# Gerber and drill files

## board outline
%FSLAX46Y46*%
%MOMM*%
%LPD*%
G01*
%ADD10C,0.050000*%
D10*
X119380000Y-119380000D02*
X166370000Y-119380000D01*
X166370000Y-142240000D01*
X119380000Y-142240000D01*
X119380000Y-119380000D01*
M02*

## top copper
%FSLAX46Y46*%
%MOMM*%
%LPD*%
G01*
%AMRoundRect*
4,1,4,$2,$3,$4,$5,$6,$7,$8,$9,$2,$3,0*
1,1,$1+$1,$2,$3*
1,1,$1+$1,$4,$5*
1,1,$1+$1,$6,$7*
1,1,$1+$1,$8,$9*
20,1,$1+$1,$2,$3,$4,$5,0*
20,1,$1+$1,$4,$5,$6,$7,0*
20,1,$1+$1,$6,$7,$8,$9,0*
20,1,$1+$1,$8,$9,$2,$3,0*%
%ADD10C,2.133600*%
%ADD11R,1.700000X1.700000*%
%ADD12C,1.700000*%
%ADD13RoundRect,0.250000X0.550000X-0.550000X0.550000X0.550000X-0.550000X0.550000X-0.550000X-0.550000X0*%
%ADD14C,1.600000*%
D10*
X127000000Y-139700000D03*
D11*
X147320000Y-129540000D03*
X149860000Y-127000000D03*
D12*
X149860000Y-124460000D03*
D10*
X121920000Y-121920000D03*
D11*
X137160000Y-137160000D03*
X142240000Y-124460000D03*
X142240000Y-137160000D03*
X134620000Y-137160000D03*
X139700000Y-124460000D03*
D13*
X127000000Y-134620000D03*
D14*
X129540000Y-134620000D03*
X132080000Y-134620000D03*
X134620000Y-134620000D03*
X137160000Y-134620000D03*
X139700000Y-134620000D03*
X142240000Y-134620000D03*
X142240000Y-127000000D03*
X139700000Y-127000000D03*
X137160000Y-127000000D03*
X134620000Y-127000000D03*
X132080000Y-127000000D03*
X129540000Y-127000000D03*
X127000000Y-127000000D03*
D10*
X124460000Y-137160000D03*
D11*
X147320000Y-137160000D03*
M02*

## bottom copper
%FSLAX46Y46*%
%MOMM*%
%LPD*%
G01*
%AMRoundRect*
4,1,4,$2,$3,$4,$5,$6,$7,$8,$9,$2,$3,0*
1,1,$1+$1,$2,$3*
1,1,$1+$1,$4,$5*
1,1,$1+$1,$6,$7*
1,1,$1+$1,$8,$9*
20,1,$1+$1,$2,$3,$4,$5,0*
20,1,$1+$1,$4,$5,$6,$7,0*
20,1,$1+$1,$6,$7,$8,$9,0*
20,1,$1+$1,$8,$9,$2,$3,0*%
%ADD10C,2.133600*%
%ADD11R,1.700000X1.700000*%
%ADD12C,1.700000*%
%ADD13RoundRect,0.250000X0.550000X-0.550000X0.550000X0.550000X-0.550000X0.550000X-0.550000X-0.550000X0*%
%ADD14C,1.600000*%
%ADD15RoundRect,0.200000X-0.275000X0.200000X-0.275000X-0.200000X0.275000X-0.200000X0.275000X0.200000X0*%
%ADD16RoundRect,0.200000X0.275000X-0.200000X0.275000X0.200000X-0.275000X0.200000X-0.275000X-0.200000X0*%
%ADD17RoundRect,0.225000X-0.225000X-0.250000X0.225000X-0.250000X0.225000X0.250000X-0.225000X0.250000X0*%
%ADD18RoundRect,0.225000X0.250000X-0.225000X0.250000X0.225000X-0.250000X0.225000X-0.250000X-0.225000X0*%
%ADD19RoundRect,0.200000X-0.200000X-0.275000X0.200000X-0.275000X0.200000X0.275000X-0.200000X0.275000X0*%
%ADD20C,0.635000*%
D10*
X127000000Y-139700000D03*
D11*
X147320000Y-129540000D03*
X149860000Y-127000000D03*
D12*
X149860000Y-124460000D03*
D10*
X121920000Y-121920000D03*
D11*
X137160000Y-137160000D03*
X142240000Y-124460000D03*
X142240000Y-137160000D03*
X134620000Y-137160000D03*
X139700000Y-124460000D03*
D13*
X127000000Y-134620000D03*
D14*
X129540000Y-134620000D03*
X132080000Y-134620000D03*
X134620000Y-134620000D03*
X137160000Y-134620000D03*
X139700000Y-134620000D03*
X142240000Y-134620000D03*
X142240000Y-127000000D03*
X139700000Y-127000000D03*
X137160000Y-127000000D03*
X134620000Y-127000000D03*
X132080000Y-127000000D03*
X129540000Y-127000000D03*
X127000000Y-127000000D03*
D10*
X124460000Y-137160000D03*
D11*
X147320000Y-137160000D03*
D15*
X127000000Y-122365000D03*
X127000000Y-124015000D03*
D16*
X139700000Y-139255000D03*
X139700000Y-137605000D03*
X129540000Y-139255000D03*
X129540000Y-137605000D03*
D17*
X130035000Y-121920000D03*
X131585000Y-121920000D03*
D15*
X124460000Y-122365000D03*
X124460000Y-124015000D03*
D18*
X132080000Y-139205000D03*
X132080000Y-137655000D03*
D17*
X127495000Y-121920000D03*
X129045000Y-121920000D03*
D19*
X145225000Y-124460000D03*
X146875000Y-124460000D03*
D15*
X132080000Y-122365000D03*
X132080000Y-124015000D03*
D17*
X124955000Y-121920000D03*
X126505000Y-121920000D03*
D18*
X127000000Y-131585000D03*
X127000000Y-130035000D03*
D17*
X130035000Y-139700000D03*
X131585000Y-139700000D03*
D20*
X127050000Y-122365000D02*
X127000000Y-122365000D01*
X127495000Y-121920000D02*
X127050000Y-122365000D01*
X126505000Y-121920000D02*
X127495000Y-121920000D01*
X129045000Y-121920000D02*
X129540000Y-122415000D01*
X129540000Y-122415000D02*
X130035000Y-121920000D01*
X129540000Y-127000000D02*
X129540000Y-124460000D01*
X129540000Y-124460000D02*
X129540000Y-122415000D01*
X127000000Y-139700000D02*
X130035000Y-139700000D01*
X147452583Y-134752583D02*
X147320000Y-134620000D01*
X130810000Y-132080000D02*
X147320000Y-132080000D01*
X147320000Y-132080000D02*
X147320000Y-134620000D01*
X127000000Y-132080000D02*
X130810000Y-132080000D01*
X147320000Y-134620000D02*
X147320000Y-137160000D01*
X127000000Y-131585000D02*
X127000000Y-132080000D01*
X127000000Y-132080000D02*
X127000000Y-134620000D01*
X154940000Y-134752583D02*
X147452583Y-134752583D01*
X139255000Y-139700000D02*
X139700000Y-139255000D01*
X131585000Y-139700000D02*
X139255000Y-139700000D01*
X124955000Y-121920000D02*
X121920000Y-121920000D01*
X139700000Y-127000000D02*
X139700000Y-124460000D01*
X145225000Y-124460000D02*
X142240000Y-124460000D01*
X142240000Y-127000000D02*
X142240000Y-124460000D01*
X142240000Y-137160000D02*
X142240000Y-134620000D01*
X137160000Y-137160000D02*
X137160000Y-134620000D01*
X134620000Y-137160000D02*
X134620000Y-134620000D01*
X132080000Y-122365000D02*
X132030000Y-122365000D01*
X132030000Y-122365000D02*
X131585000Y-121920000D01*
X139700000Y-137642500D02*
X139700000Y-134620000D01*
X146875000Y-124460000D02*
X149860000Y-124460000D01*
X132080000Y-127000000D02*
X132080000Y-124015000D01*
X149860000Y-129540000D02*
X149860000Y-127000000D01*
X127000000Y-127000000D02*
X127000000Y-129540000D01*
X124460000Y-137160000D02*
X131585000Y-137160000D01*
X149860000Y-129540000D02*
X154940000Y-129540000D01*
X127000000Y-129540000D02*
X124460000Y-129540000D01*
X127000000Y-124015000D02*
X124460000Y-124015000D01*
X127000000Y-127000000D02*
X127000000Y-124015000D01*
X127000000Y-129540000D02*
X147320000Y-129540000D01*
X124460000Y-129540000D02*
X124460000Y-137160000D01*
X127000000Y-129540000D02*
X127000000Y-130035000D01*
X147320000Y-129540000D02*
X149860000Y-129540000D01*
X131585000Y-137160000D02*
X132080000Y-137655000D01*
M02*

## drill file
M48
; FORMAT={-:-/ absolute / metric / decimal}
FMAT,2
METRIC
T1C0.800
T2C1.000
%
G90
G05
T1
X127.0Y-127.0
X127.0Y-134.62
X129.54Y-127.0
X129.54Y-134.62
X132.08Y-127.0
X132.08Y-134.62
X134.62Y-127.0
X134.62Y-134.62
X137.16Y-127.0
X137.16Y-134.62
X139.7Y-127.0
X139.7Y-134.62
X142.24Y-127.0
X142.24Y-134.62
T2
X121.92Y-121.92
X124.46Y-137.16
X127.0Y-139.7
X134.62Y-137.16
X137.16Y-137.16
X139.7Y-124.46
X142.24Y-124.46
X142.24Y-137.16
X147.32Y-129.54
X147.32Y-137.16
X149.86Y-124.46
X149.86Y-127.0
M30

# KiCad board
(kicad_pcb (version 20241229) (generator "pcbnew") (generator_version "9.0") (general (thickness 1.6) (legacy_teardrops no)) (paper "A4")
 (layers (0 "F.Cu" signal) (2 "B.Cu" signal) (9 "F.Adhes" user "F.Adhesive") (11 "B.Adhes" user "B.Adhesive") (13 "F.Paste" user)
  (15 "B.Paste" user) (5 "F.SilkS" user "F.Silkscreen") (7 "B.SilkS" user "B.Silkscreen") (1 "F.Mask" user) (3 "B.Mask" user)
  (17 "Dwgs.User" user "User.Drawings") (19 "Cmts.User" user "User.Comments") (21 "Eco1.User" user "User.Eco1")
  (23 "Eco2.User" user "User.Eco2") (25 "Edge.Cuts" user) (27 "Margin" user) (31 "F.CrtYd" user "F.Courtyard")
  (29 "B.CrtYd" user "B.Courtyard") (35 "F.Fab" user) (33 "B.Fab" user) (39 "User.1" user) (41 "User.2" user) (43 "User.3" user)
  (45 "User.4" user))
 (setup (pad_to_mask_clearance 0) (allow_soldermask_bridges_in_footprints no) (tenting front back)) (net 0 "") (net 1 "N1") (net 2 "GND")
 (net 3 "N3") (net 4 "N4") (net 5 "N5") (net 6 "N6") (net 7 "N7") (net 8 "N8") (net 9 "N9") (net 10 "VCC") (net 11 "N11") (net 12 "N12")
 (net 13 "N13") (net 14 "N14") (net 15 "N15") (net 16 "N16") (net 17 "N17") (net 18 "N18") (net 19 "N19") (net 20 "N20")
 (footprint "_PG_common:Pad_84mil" (layer "F.Cu") (at 127 139.7)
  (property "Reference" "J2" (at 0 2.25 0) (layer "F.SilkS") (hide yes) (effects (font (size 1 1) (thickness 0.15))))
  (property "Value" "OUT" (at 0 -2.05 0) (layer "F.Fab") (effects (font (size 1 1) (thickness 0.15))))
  (pad "1" thru_hole circle (at 0 0) (size 2.1336 2.1336) (drill 1) (layers "*.Cu" "*.Mask") (remove_unused_layers no) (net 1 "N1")))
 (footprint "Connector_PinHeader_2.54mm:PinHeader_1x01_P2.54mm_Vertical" (layer "F.Cu") (at 147.32 129.54)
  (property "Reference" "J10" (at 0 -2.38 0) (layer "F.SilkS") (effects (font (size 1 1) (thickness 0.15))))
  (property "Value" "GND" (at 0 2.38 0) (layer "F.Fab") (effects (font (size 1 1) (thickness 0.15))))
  (pad "1" thru_hole rect (at 0 0) (size 1.7 1.7) (drill 1) (layers "*.Cu" "*.Mask") (remove_unused_layers no) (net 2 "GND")))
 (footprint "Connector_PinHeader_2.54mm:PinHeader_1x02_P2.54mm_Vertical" (layer "F.Cu") (at 149.86 127 180)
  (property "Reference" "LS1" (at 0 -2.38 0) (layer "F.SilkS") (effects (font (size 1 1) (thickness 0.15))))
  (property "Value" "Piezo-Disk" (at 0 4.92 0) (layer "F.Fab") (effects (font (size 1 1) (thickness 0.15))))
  (pad "1" thru_hole rect (at 0 0 180) (size 1.7 1.7) (drill 1) (layers "*.Cu" "*.Mask") (remove_unused_layers no) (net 2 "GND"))
  (pad "2" thru_hole circle (at 0 2.54 180) (size 1.7 1.7) (drill 1) (layers "*.Cu" "*.Mask") (remove_unused_layers no) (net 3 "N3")))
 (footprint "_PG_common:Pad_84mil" (layer "F.Cu") (at 121.92 121.92)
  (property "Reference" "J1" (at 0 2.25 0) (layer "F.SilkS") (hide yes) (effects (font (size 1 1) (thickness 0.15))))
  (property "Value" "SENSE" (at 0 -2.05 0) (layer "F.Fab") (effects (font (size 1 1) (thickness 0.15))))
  (pad "1" thru_hole circle (at 0 0) (size 2.1336 2.1336) (drill 1) (layers "*.Cu" "*.Mask") (remove_unused_layers no) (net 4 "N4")))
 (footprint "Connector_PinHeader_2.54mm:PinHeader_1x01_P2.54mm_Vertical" (layer "F.Cu") (at 137.16 137.16)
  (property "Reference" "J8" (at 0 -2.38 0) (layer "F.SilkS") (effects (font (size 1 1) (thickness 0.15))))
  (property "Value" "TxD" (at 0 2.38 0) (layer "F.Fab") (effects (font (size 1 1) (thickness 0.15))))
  (pad "1" thru_hole rect (at 0 0) (size 1.7 1.7) (drill 1) (layers "*.Cu" "*.Mask") (remove_unused_layers no) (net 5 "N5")))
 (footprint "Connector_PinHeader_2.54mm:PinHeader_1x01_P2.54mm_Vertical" (layer "F.Cu") (at 142.24 124.46)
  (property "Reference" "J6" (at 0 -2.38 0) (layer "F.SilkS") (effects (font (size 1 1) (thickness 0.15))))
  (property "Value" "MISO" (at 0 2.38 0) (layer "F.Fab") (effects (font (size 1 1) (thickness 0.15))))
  (pad "1" thru_hole rect (at 0 0) (size 1.7 1.7) (drill 1) (layers "*.Cu" "*.Mask") (remove_unused_layers no) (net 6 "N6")))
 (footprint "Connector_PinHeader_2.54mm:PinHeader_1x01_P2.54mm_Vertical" (layer "F.Cu") (at 142.24 137.16)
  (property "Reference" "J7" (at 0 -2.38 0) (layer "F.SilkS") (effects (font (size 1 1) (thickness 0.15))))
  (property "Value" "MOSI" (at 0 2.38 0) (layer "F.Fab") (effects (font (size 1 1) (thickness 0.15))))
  (pad "1" thru_hole rect (at 0 0) (size 1.7 1.7) (drill 1) (layers "*.Cu" "*.Mask") (remove_unused_layers no) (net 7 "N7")))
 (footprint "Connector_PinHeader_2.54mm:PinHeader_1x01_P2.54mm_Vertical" (layer "F.Cu") (at 134.62 137.16)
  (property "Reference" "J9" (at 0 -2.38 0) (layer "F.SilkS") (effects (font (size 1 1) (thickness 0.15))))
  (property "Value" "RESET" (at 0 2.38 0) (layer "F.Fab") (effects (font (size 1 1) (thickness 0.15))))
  (pad "1" thru_hole rect (at 0 0) (size 1.7 1.7) (drill 1) (layers "*.Cu" "*.Mask") (remove_unused_layers no) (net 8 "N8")))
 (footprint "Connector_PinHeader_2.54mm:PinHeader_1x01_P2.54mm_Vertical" (layer "F.Cu") (at 139.7 124.46)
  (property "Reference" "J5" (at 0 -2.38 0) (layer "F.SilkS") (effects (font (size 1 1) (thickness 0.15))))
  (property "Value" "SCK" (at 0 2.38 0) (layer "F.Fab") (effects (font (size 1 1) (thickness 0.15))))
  (pad "1" thru_hole rect (at 0 0) (size 1.7 1.7) (drill 1) (layers "*.Cu" "*.Mask") (remove_unused_layers no) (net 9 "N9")))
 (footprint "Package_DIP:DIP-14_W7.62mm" (layer "F.Cu") (at 127 134.62 90)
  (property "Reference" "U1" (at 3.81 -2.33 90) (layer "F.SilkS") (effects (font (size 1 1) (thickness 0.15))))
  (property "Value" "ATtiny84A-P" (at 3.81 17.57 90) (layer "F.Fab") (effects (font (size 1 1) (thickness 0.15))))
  (pad "1" thru_hole roundrect (at 0 0 90) (size 1.6 1.6) (drill 0.8) (layers "*.Cu" "*.Mask") (remove_unused_layers no)
   (roundrect_rratio 0.15625) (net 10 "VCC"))
  (pad "2" thru_hole circle (at 0 2.54 90) (size 1.6 1.6) (drill 0.8) (layers "*.Cu" "*.Mask") (remove_unused_layers no) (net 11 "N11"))
  (pad "3" thru_hole circle (at 0 5.08 90) (size 1.6 1.6) (drill 0.8) (layers "*.Cu" "*.Mask") (remove_unused_layers no) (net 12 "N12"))
  (pad "4" thru_hole circle (at 0 7.62 90) (size 1.6 1.6) (drill 0.8) (layers "*.Cu" "*.Mask") (remove_unused_layers no) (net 8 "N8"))
  (pad "5" thru_hole circle (at 0 10.16 90) (size 1.6 1.6) (drill 0.8) (layers "*.Cu" "*.Mask") (remove_unused_layers no) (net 5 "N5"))
  (pad "6" thru_hole circle (at 0 12.7 90) (size 1.6 1.6) (drill 0.8) (layers "*.Cu" "*.Mask") (remove_unused_layers no) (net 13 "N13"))
  (pad "7" thru_hole circle (at 0 15.24 90) (size 1.6 1.6) (drill 0.8) (layers "*.Cu" "*.Mask") (remove_unused_layers no) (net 7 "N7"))
  (pad "8" thru_hole circle (at 7.62 15.24 90) (size 1.6 1.6) (drill 0.8) (layers "*.Cu" "*.Mask") (remove_unused_layers no) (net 6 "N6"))
  (pad "9" thru_hole circle (at 7.62 12.7 90) (size 1.6 1.6) (drill 0.8) (layers "*.Cu" "*.Mask") (remove_unused_layers no) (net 9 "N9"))
  (pad "10" thru_hole circle (at 7.62 10.16 90) (size 1.6 1.6) (drill 0.8) (layers "*.Cu" "*.Mask") (remove_unused_layers no) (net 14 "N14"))
  (pad "11" thru_hole circle (at 7.62 7.62 90) (size 1.6 1.6) (drill 0.8) (layers "*.Cu" "*.Mask") (remove_unused_layers no) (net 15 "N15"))
  (pad "12" thru_hole circle (at 7.62 5.08 90) (size 1.6 1.6) (drill 0.8) (layers "*.Cu" "*.Mask") (remove_unused_layers no) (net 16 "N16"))
  (pad "13" thru_hole circle (at 7.62 2.54 90) (size 1.6 1.6) (drill 0.8) (layers "*.Cu" "*.Mask") (remove_unused_layers no) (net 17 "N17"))
  (pad "14" thru_hole circle (at 7.62 0 90) (size 1.6 1.6) (drill 0.8) (layers "*.Cu" "*.Mask") (remove_unused_layers no) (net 2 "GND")))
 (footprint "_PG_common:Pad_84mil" (layer "F.Cu") (at 124.46 137.16)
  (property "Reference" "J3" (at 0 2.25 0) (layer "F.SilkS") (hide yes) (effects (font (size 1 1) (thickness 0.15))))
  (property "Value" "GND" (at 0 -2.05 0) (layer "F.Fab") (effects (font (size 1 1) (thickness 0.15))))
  (pad "1" thru_hole circle (at 0 0) (size 2.1336 2.1336) (drill 1) (layers "*.Cu" "*.Mask") (remove_unused_layers no) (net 2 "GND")))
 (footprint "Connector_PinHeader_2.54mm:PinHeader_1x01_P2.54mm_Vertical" (layer "F.Cu") (at 147.32 137.16)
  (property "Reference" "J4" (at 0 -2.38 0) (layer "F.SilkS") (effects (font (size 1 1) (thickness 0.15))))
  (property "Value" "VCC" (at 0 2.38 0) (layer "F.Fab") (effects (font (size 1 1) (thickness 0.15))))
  (pad "1" thru_hole rect (at 0 0) (size 1.7 1.7) (drill 1) (layers "*.Cu" "*.Mask") (remove_unused_layers no) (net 10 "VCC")))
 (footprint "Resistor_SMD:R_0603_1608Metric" (layer "B.Cu") (at 127 123.19 -90)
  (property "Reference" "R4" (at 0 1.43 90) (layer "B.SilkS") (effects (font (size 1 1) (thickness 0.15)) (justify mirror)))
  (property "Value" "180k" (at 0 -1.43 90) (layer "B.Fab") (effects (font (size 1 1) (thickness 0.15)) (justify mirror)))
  (pad "1" smd roundrect (at -0.825 0 270) (size 0.8 0.95) (layers "B.Cu" "B.Mask" "B.Paste") (roundrect_rratio 0.25) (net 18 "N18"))
  (pad "2" smd roundrect (at 0.825 0 270) (size 0.8 0.95) (layers "B.Cu" "B.Mask" "B.Paste") (roundrect_rratio 0.25) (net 2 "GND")))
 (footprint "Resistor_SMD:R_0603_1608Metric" (layer "B.Cu") (at 139.7 138.43 90)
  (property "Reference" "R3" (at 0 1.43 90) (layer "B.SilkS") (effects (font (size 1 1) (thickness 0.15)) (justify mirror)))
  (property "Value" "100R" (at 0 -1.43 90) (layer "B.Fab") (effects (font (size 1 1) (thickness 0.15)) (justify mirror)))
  (pad "1" smd roundrect (at -0.825 0 90) (size 0.8 0.95) (layers "B.Cu" "B.Mask" "B.Paste") (roundrect_rratio 0.25) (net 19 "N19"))
  (pad "2" smd roundrect (at 0.825 0 90) (size 0.8 0.95) (layers "B.Cu" "B.Mask" "B.Paste") (roundrect_rratio 0.25) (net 13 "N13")))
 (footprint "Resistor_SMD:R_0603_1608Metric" (layer "B.Cu") (at 129.54 138.43 90)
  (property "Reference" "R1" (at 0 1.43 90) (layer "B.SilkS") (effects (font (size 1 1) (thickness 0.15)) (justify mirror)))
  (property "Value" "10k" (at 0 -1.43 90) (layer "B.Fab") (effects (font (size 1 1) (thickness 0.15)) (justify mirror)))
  (pad "1" smd roundrect (at -0.825 0 90) (size 0.8 0.95) (layers "B.Cu" "B.Mask" "B.Paste") (roundrect_rratio 0.25) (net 1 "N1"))
  (pad "2" smd roundrect (at 0.825 0 90) (size 0.8 0.95) (layers "B.Cu" "B.Mask" "B.Paste") (roundrect_rratio 0.25) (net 2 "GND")))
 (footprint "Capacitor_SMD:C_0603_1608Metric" (layer "B.Cu") (at 130.81 121.92)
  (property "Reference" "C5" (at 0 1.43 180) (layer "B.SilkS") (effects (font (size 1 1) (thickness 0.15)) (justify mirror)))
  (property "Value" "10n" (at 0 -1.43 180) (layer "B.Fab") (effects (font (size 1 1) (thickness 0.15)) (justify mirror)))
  (pad "1" smd roundrect (at -0.775 0) (size 0.9 0.95) (layers "B.Cu" "B.Mask" "B.Paste") (roundrect_rratio 0.25) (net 17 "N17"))
  (pad "2" smd roundrect (at 0.775 0) (size 0.9 0.95) (layers "B.Cu" "B.Mask" "B.Paste") (roundrect_rratio 0.25) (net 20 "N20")))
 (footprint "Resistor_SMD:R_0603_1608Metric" (layer "B.Cu") (at 124.46 123.19 -90)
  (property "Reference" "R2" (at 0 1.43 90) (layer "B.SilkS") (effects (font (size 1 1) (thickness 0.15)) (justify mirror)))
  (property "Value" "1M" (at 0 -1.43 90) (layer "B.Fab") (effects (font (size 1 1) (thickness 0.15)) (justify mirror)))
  (pad "1" smd roundrect (at -0.825 0 270) (size 0.8 0.95) (layers "B.Cu" "B.Mask" "B.Paste") (roundrect_rratio 0.25) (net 4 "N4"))
  (pad "2" smd roundrect (at 0.825 0 270) (size 0.8 0.95) (layers "B.Cu" "B.Mask" "B.Paste") (roundrect_rratio 0.25) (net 2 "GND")))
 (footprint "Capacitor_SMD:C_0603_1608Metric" (layer "B.Cu") (at 132.08 138.43 90)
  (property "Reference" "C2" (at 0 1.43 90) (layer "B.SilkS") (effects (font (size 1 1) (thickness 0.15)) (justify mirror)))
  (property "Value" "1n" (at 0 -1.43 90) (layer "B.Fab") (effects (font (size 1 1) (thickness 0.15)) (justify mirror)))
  (pad "1" smd roundrect (at -0.775 0 90) (size 0.9 0.95) (layers "B.Cu" "B.Mask" "B.Paste") (roundrect_rratio 0.25) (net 19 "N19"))
  (pad "2" smd roundrect (at 0.775 0 90) (size 0.9 0.95) (layers "B.Cu" "B.Mask" "B.Paste") (roundrect_rratio 0.25) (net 2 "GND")))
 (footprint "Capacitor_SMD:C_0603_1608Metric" (layer "B.Cu") (at 128.27 121.92)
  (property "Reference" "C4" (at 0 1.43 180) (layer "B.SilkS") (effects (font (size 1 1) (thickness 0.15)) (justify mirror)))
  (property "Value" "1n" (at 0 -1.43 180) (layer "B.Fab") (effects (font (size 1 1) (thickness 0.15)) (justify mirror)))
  (pad "1" smd roundrect (at -0.775 0) (size 0.9 0.95) (layers "B.Cu" "B.Mask" "B.Paste") (roundrect_rratio 0.25) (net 18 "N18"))
  (pad "2" smd roundrect (at 0.775 0) (size 0.9 0.95) (layers "B.Cu" "B.Mask" "B.Paste") (roundrect_rratio 0.25) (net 17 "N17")))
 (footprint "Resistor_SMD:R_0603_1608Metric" (layer "B.Cu") (at 146.05 124.46)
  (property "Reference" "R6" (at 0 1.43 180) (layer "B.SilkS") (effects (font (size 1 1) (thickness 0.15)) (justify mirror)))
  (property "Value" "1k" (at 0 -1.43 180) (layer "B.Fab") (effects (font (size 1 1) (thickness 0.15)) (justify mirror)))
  (pad "1" smd roundrect (at -0.825 0) (size 0.8 0.95) (layers "B.Cu" "B.Mask" "B.Paste") (roundrect_rratio 0.25) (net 6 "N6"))
  (pad "2" smd roundrect (at 0.825 0) (size 0.8 0.95) (layers "B.Cu" "B.Mask" "B.Paste") (roundrect_rratio 0.25) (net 3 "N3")))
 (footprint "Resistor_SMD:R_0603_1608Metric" (layer "B.Cu") (at 132.08 123.19 -90)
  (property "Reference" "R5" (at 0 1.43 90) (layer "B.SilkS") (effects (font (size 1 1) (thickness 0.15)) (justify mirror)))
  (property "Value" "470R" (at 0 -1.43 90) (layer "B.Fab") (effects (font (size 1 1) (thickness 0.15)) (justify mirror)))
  (pad "1" smd roundrect (at -0.825 0 270) (size 0.8 0.95) (layers "B.Cu" "B.Mask" "B.Paste") (roundrect_rratio 0.25) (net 20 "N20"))
  (pad "2" smd roundrect (at 0.825 0 270) (size 0.8 0.95) (layers "B.Cu" "B.Mask" "B.Paste") (roundrect_rratio 0.25) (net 16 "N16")))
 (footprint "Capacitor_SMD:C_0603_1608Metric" (layer "B.Cu") (at 125.73 121.92)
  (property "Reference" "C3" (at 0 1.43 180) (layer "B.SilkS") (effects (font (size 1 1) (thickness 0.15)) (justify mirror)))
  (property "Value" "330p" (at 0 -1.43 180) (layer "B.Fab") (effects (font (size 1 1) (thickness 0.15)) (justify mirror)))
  (pad "1" smd roundrect (at -0.775 0) (size 0.9 0.95) (layers "B.Cu" "B.Mask" "B.Paste") (roundrect_rratio 0.25) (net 4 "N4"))
  (pad "2" smd roundrect (at 0.775 0) (size 0.9 0.95) (layers "B.Cu" "B.Mask" "B.Paste") (roundrect_rratio 0.25) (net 18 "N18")))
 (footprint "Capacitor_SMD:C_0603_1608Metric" (layer "B.Cu") (at 127 130.81 90)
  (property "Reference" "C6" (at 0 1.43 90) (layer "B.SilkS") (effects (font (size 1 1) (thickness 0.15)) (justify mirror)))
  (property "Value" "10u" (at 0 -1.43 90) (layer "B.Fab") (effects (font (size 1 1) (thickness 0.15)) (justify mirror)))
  (pad "1" smd roundrect (at -0.775 0 90) (size 0.9 0.95) (layers "B.Cu" "B.Mask" "B.Paste") (roundrect_rratio 0.25) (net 10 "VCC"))
  (pad "2" smd roundrect (at 0.775 0 90) (size 0.9 0.95) (layers "B.Cu" "B.Mask" "B.Paste") (roundrect_rratio 0.25) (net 2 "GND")))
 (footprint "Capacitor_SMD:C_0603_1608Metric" (layer "B.Cu") (at 130.81 139.7)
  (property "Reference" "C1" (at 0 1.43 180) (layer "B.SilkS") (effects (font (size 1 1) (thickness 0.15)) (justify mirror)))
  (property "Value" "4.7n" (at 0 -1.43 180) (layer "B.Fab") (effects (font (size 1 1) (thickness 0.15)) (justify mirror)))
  (pad "1" smd roundrect (at -0.775 0) (size 0.9 0.95) (layers "B.Cu" "B.Mask" "B.Paste") (roundrect_rratio 0.25) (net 1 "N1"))
  (pad "2" smd roundrect (at 0.775 0) (size 0.9 0.95) (layers "B.Cu" "B.Mask" "B.Paste") (roundrect_rratio 0.25) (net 19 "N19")))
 (gr_rect (start 119.38 119.38) (end 166.37 142.24) (stroke (width 0.05) (type default)) (fill no) (layer "Edge.Cuts"))
 (segment (start 127.05 122.365) (end 127 122.365) (width 0.635) (layer "B.Cu") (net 18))
 (segment (start 127.495 121.92) (end 127.05 122.365) (width 0.635) (layer "B.Cu") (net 18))
 (segment (start 126.505 121.92) (end 127.495 121.92) (width 0.635) (layer "B.Cu") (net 18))
 (segment (start 129.045 121.92) (end 129.54 122.415) (width 0.635) (layer "B.Cu") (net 17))
 (segment (start 129.54 122.415) (end 130.035 121.92) (width 0.635) (layer "B.Cu") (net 17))
 (segment (start 129.54 127) (end 129.54 124.46) (width 0.635) (layer "B.Cu") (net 17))
 (segment (start 129.54 124.46) (end 129.54 122.415) (width 0.635) (layer "B.Cu") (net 17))
 (segment (start 127 139.7) (end 130.035 139.7) (width 0.635) (layer "B.Cu") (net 1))
 (segment (start 147.452583 134.752583) (end 147.32 134.62) (width 0.635) (layer "B.Cu") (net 10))
 (segment (start 130.81 132.08) (end 147.32 132.08) (width 0.635) (layer "B.Cu") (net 10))
 (segment (start 147.32 132.08) (end 147.32 134.62) (width 0.635) (layer "B.Cu") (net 10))
 (segment (start 127 132.08) (end 130.81 132.08) (width 0.635) (layer "B.Cu") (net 10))
 (segment (start 147.32 134.62) (end 147.32 137.16) (width 0.635) (layer "B.Cu") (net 10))
 (segment (start 127 131.585) (end 127 132.08) (width 0.635) (layer "B.Cu") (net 10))
 (segment (start 127 132.08) (end 127 134.62) (width 0.635) (layer "B.Cu") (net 10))
 (segment (start 154.94 134.752583) (end 147.452583 134.752583) (width 0.635) (layer "B.Cu") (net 10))
 (segment (start 139.255 139.7) (end 139.7 139.255) (width 0.635) (layer "B.Cu") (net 19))
 (segment (start 131.585 139.7) (end 139.255 139.7) (width 0.635) (layer "B.Cu") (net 19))
 (segment (start 124.955 121.92) (end 121.92 121.92) (width 0.635) (layer "B.Cu") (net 4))
 (segment (start 139.7 127) (end 139.7 124.46) (width 0.635) (layer "B.Cu") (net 9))
 (segment (start 145.225 124.46) (end 142.24 124.46) (width 0.635) (layer "B.Cu") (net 6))
 (segment (start 142.24 127) (end 142.24 124.46) (width 0.635) (layer "B.Cu") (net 6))
 (segment (start 142.24 137.16) (end 142.24 134.62) (width 0.635) (layer "B.Cu") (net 7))
 (segment (start 137.16 137.16) (end 137.16 134.62) (width 0.635) (layer "B.Cu") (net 5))
 (segment (start 134.62 137.16) (end 134.62 134.62) (width 0.635) (layer "B.Cu") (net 8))
 (segment (start 132.08 122.365) (end 132.03 122.365) (width 0.635) (layer "B.Cu") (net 20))
 (segment (start 132.03 122.365) (end 131.585 121.92) (width 0.635) (layer "B.Cu") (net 20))
 (segment (start 139.7 137.6425) (end 139.7 134.62) (width 0.635) (layer "B.Cu") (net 13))
 (segment (start 146.875 124.46) (end 149.86 124.46) (width 0.635) (layer "B.Cu") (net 3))
 (segment (start 132.08 127) (end 132.08 124.015) (width 0.635) (layer "B.Cu") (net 16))
 (segment (start 149.86 129.54) (end 149.86 127) (width 0.635) (layer "B.Cu") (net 2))
 (segment (start 127 127) (end 127 129.54) (width 0.635) (layer "B.Cu") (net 2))
 (segment (start 124.46 137.16) (end 131.585 137.16) (width 0.635) (layer "B.Cu") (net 2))
 (segment (start 149.86 129.54) (end 154.94 129.54) (width 0.635) (layer "B.Cu") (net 2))
 (segment (start 127 129.54) (end 124.46 129.54) (width 0.635) (layer "B.Cu") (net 2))
 (segment (start 127 124.015) (end 124.46 124.015) (width 0.635) (layer "B.Cu") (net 2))
 (segment (start 127 127) (end 127 124.015) (width 0.635) (layer "B.Cu") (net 2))
 (segment (start 127 129.54) (end 147.32 129.54) (width 0.635) (layer "B.Cu") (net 2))
 (segment (start 124.46 129.54) (end 124.46 137.16) (width 0.635) (layer "B.Cu") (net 2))
 (segment (start 127 129.54) (end 127 130.035) (width 0.635) (layer "B.Cu") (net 2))
 (segment (start 147.32 129.54) (end 149.86 129.54) (width 0.635) (layer "B.Cu") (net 2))
 (segment (start 131.585 137.16) (end 132.08 137.655) (width 0.635) (layer "B.Cu") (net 2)))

